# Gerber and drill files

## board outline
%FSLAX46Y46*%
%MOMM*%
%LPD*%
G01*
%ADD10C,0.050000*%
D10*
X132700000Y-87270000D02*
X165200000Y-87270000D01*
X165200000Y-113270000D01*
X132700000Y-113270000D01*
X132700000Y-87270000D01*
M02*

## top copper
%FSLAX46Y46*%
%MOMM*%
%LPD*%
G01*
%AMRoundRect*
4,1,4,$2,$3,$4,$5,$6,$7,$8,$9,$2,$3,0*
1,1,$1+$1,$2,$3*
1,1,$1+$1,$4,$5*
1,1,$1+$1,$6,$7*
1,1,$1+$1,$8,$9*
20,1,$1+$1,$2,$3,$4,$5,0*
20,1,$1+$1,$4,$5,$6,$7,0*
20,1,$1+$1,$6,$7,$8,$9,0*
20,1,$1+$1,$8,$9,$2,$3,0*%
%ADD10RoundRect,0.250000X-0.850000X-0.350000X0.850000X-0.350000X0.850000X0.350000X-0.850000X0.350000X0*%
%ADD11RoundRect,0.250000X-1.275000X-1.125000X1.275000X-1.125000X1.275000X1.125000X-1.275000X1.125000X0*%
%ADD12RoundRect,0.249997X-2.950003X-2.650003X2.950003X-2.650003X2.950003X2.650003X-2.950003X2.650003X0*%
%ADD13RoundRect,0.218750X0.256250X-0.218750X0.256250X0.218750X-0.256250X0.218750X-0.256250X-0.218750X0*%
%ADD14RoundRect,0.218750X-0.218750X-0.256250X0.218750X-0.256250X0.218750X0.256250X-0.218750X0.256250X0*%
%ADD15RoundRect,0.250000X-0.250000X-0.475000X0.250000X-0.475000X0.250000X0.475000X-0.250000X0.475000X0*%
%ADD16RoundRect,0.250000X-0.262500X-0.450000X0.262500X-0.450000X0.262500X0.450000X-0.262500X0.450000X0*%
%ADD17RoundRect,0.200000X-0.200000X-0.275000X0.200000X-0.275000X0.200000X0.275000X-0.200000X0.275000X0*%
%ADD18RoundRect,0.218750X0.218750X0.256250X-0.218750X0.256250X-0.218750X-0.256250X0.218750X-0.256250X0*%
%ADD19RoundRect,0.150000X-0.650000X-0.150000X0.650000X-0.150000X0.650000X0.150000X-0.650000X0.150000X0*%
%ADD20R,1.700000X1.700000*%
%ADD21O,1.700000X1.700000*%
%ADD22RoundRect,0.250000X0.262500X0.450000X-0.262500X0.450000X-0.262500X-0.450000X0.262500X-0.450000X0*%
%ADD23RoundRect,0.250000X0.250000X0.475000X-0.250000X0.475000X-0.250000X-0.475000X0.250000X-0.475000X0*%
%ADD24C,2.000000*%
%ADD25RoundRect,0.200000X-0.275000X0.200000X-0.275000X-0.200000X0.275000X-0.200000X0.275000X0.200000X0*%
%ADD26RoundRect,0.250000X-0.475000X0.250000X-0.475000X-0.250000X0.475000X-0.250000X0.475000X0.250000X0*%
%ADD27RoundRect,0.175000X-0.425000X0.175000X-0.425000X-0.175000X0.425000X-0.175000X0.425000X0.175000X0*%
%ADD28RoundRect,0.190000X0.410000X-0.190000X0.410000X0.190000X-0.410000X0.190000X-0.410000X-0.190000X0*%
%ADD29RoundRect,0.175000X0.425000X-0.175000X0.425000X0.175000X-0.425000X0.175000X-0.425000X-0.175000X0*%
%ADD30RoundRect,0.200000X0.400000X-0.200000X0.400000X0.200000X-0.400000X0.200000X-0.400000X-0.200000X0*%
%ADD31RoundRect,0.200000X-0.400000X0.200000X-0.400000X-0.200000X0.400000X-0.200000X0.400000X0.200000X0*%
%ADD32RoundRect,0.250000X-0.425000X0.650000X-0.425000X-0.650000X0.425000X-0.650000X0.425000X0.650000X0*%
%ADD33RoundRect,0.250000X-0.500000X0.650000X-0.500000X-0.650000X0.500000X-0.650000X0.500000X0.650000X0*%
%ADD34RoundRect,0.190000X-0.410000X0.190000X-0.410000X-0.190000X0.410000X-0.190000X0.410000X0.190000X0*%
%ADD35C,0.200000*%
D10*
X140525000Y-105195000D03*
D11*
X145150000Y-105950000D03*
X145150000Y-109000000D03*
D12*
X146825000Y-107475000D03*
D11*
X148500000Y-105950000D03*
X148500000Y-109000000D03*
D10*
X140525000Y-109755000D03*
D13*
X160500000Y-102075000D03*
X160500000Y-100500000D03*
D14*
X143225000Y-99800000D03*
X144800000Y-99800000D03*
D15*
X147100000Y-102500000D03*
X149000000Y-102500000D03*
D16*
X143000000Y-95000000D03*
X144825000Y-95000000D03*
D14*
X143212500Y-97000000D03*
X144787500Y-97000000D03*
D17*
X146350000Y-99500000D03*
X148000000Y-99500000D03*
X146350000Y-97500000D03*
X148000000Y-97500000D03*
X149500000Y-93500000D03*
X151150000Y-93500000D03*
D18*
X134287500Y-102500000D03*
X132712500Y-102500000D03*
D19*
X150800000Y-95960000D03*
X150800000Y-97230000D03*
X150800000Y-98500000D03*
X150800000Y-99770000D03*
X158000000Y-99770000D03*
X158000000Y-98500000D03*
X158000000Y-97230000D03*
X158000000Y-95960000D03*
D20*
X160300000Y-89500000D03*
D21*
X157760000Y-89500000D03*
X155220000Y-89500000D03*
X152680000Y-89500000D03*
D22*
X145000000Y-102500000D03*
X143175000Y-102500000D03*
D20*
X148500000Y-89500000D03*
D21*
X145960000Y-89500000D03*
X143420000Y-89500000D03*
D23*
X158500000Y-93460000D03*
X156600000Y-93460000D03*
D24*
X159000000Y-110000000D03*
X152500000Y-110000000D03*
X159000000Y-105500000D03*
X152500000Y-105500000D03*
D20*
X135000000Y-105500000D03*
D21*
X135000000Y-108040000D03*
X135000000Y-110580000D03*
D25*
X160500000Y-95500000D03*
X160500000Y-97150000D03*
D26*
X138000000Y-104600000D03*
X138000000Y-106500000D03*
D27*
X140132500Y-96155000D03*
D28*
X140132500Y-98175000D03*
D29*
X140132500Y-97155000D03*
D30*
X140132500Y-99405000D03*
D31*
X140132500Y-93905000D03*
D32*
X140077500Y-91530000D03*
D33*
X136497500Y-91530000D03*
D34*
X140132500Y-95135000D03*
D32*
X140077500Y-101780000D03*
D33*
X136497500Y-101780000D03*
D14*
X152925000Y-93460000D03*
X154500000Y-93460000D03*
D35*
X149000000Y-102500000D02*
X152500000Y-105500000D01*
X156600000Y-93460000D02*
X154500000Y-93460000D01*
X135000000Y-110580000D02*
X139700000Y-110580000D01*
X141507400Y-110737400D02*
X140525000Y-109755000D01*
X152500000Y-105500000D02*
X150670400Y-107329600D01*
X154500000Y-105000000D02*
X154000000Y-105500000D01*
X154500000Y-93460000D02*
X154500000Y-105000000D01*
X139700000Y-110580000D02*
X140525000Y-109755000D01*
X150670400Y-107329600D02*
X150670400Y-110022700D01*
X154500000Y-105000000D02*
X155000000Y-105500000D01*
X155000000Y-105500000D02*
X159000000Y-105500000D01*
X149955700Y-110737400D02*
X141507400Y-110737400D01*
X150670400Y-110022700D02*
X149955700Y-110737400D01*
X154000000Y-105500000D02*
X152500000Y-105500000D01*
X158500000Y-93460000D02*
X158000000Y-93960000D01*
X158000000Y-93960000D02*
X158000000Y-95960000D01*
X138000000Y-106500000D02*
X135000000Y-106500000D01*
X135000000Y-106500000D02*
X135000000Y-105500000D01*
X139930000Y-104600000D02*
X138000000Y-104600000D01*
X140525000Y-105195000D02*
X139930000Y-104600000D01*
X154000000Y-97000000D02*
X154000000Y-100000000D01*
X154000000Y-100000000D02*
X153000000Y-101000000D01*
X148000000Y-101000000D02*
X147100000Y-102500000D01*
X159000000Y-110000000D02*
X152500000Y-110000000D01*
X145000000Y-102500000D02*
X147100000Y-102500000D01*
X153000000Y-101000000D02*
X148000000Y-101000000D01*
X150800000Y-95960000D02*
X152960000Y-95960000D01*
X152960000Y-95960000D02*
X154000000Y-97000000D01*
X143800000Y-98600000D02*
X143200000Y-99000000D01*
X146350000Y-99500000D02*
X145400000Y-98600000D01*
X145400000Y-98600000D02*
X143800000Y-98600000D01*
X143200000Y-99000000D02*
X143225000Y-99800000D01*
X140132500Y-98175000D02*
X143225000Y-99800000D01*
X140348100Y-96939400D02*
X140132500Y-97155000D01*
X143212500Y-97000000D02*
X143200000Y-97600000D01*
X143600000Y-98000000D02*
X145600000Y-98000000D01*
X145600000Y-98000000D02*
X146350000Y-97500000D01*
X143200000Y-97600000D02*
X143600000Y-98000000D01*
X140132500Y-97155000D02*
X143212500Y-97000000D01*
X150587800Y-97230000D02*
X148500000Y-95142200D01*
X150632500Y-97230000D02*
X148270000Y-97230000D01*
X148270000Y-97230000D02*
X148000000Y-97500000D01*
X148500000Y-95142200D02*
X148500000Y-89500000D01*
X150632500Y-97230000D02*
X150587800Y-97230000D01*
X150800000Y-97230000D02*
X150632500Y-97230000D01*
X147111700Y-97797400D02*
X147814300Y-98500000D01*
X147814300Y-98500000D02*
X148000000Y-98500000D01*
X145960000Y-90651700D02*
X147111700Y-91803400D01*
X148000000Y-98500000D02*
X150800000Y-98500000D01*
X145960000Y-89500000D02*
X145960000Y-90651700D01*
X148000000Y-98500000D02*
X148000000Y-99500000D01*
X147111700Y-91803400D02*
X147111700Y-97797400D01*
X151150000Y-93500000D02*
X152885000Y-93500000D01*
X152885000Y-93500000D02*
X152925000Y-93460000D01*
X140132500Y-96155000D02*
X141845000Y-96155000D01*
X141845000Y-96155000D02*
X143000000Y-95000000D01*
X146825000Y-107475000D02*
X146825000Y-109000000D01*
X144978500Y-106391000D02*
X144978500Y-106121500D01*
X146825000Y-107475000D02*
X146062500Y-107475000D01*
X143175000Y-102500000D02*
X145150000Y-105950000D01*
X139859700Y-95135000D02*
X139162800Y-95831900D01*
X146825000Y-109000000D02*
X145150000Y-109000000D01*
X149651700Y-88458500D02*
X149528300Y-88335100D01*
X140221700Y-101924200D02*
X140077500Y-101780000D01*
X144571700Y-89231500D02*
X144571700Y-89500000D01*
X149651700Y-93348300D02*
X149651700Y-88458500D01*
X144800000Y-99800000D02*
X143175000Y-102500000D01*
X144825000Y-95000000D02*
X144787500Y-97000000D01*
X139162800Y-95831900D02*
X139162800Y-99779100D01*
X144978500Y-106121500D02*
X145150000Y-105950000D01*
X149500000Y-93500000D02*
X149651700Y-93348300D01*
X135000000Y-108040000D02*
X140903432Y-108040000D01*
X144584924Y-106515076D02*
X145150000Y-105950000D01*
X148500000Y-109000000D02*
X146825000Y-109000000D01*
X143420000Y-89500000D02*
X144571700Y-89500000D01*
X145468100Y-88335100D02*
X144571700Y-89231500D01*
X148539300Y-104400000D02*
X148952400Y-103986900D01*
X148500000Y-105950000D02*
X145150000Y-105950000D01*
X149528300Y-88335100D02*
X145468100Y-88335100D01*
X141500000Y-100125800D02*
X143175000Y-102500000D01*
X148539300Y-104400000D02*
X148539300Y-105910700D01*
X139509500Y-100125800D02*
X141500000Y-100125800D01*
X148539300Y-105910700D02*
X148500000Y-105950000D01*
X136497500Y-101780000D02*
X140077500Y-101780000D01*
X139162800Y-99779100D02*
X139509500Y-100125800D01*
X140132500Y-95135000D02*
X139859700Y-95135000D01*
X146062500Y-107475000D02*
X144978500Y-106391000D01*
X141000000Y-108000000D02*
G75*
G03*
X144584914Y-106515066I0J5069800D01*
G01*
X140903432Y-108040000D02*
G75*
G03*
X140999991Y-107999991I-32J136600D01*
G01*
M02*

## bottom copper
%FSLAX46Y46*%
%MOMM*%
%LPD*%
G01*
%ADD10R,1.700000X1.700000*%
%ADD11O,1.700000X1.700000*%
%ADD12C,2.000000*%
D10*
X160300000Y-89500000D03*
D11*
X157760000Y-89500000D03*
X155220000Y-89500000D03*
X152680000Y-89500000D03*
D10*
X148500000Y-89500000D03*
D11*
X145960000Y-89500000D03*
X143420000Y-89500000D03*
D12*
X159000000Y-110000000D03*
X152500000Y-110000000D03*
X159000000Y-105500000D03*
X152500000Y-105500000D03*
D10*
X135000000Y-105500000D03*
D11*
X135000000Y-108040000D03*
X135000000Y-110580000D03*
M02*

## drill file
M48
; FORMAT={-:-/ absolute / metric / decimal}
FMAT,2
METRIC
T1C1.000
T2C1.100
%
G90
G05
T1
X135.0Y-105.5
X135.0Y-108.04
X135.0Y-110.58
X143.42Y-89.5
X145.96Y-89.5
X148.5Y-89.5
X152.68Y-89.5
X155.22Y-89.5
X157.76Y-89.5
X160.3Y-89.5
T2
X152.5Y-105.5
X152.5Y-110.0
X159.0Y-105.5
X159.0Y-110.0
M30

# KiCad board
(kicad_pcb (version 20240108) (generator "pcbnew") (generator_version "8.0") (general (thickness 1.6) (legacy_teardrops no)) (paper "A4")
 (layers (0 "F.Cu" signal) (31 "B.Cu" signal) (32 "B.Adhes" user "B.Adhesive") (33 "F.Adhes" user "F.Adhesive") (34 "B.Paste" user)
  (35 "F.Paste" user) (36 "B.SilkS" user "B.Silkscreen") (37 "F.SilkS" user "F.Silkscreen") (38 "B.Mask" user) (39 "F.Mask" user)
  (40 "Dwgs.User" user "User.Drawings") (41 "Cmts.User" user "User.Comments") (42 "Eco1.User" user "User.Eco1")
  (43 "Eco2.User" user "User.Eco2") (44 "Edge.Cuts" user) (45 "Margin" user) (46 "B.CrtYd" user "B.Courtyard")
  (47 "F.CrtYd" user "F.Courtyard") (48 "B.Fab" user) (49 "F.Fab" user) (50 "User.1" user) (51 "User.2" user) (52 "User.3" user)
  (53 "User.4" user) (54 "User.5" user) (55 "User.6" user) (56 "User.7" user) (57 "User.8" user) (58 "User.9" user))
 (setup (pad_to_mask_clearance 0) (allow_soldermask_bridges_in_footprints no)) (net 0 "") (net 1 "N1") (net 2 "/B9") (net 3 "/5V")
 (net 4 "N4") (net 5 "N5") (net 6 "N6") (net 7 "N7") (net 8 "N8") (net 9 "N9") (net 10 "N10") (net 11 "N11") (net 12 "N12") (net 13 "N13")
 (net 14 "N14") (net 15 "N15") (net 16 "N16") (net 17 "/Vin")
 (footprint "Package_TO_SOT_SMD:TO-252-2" (layer "F.Cu") (at 145.565 107.475)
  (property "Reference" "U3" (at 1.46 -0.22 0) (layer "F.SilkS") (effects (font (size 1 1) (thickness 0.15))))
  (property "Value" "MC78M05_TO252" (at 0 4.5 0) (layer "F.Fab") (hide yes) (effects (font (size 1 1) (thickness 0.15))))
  (pad "1" smd roundrect (at -5.04 -2.28) (size 2.2 1.2) (layers "F.Cu" "F.Paste" "F.Mask") (roundrect_rratio 0.208333) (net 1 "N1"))
  (pad "2" smd roundrect (at -0.415 -1.525) (size 3.05 2.75) (layers "F.Cu" "F.Paste") (roundrect_rratio 0.090909) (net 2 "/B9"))
  (pad "2" smd roundrect (at -0.415 1.525) (size 3.05 2.75) (layers "F.Cu" "F.Paste") (roundrect_rratio 0.090909) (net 2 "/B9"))
  (pad "2" smd roundrect (at 1.26 0) (size 6.4 5.8) (layers "F.Cu" "F.Mask") (roundrect_rratio 0.043103) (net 2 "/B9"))
  (pad "2" smd roundrect (at 2.935 -1.525) (size 3.05 2.75) (layers "F.Cu" "F.Paste") (roundrect_rratio 0.090909) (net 2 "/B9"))
  (pad "2" smd roundrect (at 2.935 1.525) (size 3.05 2.75) (layers "F.Cu" "F.Paste") (roundrect_rratio 0.090909) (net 2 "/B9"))
  (pad "3" smd roundrect (at -5.04 2.28) (size 2.2 1.2) (layers "F.Cu" "F.Paste" "F.Mask") (roundrect_rratio 0.208333) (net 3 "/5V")))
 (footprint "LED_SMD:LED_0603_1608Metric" (layer "F.Cu") (at 160.5 101.2875 90)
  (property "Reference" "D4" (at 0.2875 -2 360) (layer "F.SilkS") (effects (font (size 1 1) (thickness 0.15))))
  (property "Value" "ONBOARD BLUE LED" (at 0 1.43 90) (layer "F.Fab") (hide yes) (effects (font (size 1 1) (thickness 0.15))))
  (pad "1" smd roundrect (at -0.7875 0 90) (size 0.875 0.95) (layers "F.Cu" "F.Paste" "F.Mask") (roundrect_rratio 0.25) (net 2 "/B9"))
  (pad "2" smd roundrect (at 0.7875 0 90) (size 0.875 0.95) (layers "F.Cu" "F.Paste" "F.Mask") (roundrect_rratio 0.25) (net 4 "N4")))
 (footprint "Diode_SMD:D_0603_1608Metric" (layer "F.Cu") (at 144.0125 99.8)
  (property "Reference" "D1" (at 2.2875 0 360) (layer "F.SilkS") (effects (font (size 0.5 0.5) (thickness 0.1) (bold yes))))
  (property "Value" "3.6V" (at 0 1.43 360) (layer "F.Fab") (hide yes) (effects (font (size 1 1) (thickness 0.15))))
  (pad "1" smd roundrect (at -0.7875 0) (size 0.875 0.95) (layers "F.Cu" "F.Paste" "F.Mask") (roundrect_rratio 0.25) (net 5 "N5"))
  (pad "2" smd roundrect (at 0.7875 0) (size 0.875 0.95) (layers "F.Cu" "F.Paste" "F.Mask") (roundrect_rratio 0.25) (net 2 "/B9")))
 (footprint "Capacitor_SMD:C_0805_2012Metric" (layer "F.Cu") (at 148.05 102.5)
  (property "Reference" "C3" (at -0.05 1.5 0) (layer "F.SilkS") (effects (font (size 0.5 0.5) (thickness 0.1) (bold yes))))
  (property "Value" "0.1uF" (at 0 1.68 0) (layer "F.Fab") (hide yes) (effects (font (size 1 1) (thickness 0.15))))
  (pad "1" smd roundrect (at -0.95 0) (size 1 1.45) (layers "F.Cu" "F.Paste" "F.Mask") (roundrect_rratio 0.25) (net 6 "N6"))
  (pad "2" smd roundrect (at 0.95 0) (size 1 1.45) (layers "F.Cu" "F.Paste" "F.Mask") (roundrect_rratio 0.25) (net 3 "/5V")))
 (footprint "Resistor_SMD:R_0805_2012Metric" (layer "F.Cu") (at 143.9125 95)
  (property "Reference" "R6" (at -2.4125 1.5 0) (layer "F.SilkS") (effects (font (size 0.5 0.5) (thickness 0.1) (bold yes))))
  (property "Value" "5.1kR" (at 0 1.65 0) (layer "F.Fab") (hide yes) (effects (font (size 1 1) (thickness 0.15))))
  (pad "1" smd roundrect (at -0.9125 0) (size 1.025 1.4) (layers "F.Cu" "F.Paste" "F.Mask") (roundrect_rratio 0.243902) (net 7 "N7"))
  (pad "2" smd roundrect (at 0.9125 0) (size 1.025 1.4) (layers "F.Cu" "F.Paste" "F.Mask") (roundrect_rratio 0.243902) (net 2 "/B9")))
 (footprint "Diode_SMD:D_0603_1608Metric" (layer "F.Cu") (at 144 97)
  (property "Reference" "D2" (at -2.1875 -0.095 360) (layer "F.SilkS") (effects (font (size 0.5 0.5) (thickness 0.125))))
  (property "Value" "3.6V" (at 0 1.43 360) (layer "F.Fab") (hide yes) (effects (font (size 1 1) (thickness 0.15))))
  (pad "1" smd roundrect (at -0.7875 0) (size 0.875 0.95) (layers "F.Cu" "F.Paste" "F.Mask") (roundrect_rratio 0.25) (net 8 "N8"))
  (pad "2" smd roundrect (at 0.7875 0) (size 0.875 0.95) (layers "F.Cu" "F.Paste" "F.Mask") (roundrect_rratio 0.25) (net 2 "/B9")))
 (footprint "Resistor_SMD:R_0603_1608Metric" (layer "F.Cu") (at 147.175 99.5)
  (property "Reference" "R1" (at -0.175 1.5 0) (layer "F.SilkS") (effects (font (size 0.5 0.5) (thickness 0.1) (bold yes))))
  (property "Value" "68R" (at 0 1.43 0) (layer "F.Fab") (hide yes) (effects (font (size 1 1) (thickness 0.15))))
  (pad "1" smd roundrect (at -0.825 0) (size 0.8 0.95) (layers "F.Cu" "F.Paste" "F.Mask") (roundrect_rratio 0.25) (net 5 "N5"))
  (pad "2" smd roundrect (at 0.825 0) (size 0.8 0.95) (layers "F.Cu" "F.Paste" "F.Mask") (roundrect_rratio 0.25) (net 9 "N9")))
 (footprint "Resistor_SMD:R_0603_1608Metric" (layer "F.Cu") (at 147.175 97.5)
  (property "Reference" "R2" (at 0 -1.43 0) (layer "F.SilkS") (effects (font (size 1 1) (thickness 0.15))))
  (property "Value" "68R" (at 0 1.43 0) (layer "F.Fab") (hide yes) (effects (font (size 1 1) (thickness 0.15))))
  (pad "1" smd roundrect (at -0.825 0) (size 0.8 0.95) (layers "F.Cu" "F.Paste" "F.Mask") (roundrect_rratio 0.25) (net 8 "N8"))
  (pad "2" smd roundrect (at 0.825 0) (size 0.8 0.95) (layers "F.Cu" "F.Paste" "F.Mask") (roundrect_rratio 0.25) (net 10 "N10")))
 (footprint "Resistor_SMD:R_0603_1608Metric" (layer "F.Cu") (at 150.325 93.5)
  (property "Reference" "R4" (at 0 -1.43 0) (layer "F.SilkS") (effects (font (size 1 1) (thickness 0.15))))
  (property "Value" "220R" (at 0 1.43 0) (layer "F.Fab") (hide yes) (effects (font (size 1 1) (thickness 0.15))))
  (pad "1" smd roundrect (at -0.825 0) (size 0.8 0.95) (layers "F.Cu" "F.Paste" "F.Mask") (roundrect_rratio 0.25) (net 2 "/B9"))
  (pad "2" smd roundrect (at 0.825 0) (size 0.8 0.95) (layers "F.Cu" "F.Paste" "F.Mask") (roundrect_rratio 0.25) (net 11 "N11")))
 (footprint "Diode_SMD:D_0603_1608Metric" (layer "F.Cu") (at 133.5 102.5 180)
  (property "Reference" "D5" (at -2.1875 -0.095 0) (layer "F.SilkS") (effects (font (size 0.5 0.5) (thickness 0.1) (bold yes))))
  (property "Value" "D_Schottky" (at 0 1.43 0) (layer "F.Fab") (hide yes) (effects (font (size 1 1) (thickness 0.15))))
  (pad "1" smd roundrect (at -0.7875 0 180) (size 0.875 0.95) (layers "F.Cu" "F.Paste" "F.Mask") (roundrect_rratio 0.25) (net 1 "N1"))
  (pad "2" smd roundrect (at 0.7875 0 180) (size 0.875 0.95) (layers "F.Cu" "F.Paste" "F.Mask") (roundrect_rratio 0.25) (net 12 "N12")))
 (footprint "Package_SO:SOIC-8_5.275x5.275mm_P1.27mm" (layer "F.Cu") (at 154.4 97.865)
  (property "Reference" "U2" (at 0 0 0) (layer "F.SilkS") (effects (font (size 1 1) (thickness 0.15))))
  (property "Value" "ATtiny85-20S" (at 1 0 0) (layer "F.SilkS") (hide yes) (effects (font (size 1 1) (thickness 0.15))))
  (pad "1" smd roundrect (at -3.6 -1.905) (size 1.6 0.6) (layers "F.Cu" "F.Paste" "F.Mask") (roundrect_rratio 0.25) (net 6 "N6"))
  (pad "2" smd roundrect (at -3.6 -0.635) (size 1.6 0.6) (layers "F.Cu" "F.Paste" "F.Mask") (roundrect_rratio 0.25) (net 10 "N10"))
  (pad "3" smd roundrect (at -3.6 0.635) (size 1.6 0.6) (layers "F.Cu" "F.Paste" "F.Mask") (roundrect_rratio 0.25) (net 9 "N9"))
  (pad "4" smd roundrect (at -3.6 1.905) (size 1.6 0.6) (layers "F.Cu" "F.Paste" "F.Mask") (roundrect_rratio 0.25) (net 2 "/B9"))
  (pad "5" smd roundrect (at 3.6 1.905) (size 1.6 0.6) (layers "F.Cu" "F.Paste" "F.Mask") (roundrect_rratio 0.25) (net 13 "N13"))
  (pad "6" smd roundrect (at 3.6 0.635) (size 1.6 0.6) (layers "F.Cu" "F.Paste" "F.Mask") (roundrect_rratio 0.25) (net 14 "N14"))
  (pad "7" smd roundrect (at 3.6 -0.635) (size 1.6 0.6) (layers "F.Cu" "F.Paste" "F.Mask") (roundrect_rratio 0.25) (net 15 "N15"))
  (pad "8" smd roundrect (at 3.6 -1.905) (size 1.6 0.6) (layers "F.Cu" "F.Paste" "F.Mask") (roundrect_rratio 0.25) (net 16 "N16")))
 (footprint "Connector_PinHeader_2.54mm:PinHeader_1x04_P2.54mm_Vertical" (layer "F.Cu") (at 160.3 89.5 -90)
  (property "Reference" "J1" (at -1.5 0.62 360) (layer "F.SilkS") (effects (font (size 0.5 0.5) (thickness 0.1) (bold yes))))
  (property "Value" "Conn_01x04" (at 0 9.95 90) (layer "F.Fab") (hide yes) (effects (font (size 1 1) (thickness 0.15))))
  (pad "1" thru_hole rect (at 0 0 270) (size 1.7 1.7) (drill 1) (layers "*.Cu" "*.Mask") (remove_unused_layers no) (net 13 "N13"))
  (pad "2" thru_hole oval (at 0 2.54 270) (size 1.7 1.7) (drill 1) (layers "*.Cu" "*.Mask") (remove_unused_layers no) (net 14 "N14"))
  (pad "3" thru_hole oval (at 0 5.08 270) (size 1.7 1.7) (drill 1) (layers "*.Cu" "*.Mask") (remove_unused_layers no) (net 15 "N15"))
  (pad "4" thru_hole oval (at 0 7.62 270) (size 1.7 1.7) (drill 1) (layers "*.Cu" "*.Mask") (remove_unused_layers no) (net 2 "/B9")))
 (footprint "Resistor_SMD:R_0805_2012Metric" (layer "F.Cu") (at 144.0875 102.5 180)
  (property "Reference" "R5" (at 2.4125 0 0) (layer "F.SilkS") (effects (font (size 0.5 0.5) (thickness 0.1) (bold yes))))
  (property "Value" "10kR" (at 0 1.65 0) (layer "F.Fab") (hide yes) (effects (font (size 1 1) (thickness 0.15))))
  (pad "1" smd roundrect (at -0.9125 0 180) (size 1.025 1.4) (layers "F.Cu" "F.Paste" "F.Mask") (roundrect_rratio 0.243902) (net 6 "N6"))
  (pad "2" smd roundrect (at 0.9125 0 180) (size 1.025 1.4) (layers "F.Cu" "F.Paste" "F.Mask") (roundrect_rratio 0.243902) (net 2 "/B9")))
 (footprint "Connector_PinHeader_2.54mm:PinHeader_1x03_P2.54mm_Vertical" (layer "F.Cu") (at 148.5 89.5 -90)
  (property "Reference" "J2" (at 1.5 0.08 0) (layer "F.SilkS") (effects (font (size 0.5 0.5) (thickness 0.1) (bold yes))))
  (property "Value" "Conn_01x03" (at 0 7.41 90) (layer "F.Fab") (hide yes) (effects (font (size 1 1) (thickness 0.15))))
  (pad "1" thru_hole rect (at 0 0 270) (size 1.7 1.7) (drill 1) (layers "*.Cu" "*.Mask") (remove_unused_layers no) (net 10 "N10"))
  (pad "2" thru_hole oval (at 0 2.54 270) (size 1.7 1.7) (drill 1) (layers "*.Cu" "*.Mask") (remove_unused_layers no) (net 9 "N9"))
  (pad "3" thru_hole oval (at 0 5.08 270) (size 1.7 1.7) (drill 1) (layers "*.Cu" "*.Mask") (remove_unused_layers no) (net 2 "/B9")))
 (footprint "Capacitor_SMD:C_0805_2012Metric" (layer "F.Cu") (at 157.55 93.46 180)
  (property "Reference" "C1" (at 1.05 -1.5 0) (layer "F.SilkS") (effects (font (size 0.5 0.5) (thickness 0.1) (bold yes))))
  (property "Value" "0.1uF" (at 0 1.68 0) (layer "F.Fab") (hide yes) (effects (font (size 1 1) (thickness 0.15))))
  (pad "1" smd roundrect (at -0.95 0 180) (size 1 1.45) (layers "F.Cu" "F.Paste" "F.Mask") (roundrect_rratio 0.25) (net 16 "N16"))
  (pad "2" smd roundrect (at 0.95 0 180) (size 1 1.45) (layers "F.Cu" "F.Paste" "F.Mask") (roundrect_rratio 0.25) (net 3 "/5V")))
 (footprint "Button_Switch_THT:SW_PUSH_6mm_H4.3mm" (layer "F.Cu") (at 159 110 180)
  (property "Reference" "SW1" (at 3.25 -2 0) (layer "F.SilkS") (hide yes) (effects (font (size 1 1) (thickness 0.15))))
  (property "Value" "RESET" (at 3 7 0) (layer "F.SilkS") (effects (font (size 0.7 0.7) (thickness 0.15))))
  (pad "1" thru_hole circle (at 0 0 270) (size 2 2) (drill 1.1) (layers "*.Cu" "*.Mask") (remove_unused_layers no) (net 6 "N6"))
  (pad "1" thru_hole circle (at 6.5 0 270) (size 2 2) (drill 1.1) (layers "*.Cu" "*.Mask") (remove_unused_layers no) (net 6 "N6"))
  (pad "2" thru_hole circle (at 0 4.5 270) (size 2 2) (drill 1.1) (layers "*.Cu" "*.Mask") (remove_unused_layers no) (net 3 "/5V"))
  (pad "2" thru_hole circle (at 6.5 4.5 270) (size 2 2) (drill 1.1) (layers "*.Cu" "*.Mask") (remove_unused_layers no) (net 3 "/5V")))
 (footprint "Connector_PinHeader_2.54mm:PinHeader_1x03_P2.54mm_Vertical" (layer "F.Cu") (at 135 105.5)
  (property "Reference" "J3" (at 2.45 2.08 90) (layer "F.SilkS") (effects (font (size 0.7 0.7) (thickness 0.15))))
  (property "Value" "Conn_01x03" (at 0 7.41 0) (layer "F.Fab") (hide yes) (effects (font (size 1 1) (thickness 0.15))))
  (pad "1" thru_hole rect (at 0 0) (size 1.7 1.7) (drill 1) (layers "*.Cu" "*.Mask") (remove_unused_layers no) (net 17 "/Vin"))
  (pad "2" thru_hole oval (at 0 2.54) (size 1.7 1.7) (drill 1) (layers "*.Cu" "*.Mask") (remove_unused_layers no) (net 2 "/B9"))
  (pad "3" thru_hole oval (at 0 5.08) (size 1.7 1.7) (drill 1) (layers "*.Cu" "*.Mask") (remove_unused_layers no) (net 3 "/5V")))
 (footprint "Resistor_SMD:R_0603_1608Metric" (layer "F.Cu") (at 160.5 96.325 -90)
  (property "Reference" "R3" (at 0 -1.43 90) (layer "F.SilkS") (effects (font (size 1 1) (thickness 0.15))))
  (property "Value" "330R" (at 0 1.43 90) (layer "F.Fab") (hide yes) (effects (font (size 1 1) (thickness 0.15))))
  (pad "1" smd roundrect (at -0.825 0 270) (size 0.8 0.95) (layers "F.Cu" "F.Paste" "F.Mask") (roundrect_rratio 0.25) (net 13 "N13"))
  (pad "2" smd roundrect (at 0.825 0 270) (size 0.8 0.95) (layers "F.Cu" "F.Paste" "F.Mask") (roundrect_rratio 0.25) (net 4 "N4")))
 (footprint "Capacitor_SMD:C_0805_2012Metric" (layer "F.Cu") (at 138 105.55 -90)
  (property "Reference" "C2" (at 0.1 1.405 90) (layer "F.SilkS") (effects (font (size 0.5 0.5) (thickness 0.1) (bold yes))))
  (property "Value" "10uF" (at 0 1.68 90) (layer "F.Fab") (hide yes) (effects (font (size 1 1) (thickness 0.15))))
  (pad "1" smd roundrect (at -0.95 0 270) (size 1 1.45) (layers "F.Cu" "F.Paste" "F.Mask") (roundrect_rratio 0.25) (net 1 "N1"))
  (pad "2" smd roundrect (at 0.95 0 270) (size 1 1.45) (layers "F.Cu" "F.Paste" "F.Mask") (roundrect_rratio 0.25) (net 17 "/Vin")))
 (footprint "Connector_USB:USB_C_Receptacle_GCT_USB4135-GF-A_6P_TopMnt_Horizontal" (layer "F.Cu") (at 137.1 96.655 -90)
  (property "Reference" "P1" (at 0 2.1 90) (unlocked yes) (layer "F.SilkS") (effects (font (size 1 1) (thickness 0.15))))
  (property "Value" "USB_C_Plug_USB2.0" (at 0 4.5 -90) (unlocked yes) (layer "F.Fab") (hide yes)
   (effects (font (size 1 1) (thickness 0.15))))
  (pad "A5" smd roundrect (at -0.5 -3.0325 270) (size 0.7 1.2) (layers "F.Cu" "F.Paste" "F.Mask") (roundrect_rratio 0.25) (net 7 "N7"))
  (pad "A6" smd roundrect (at 1.52 -3.0325 90) (size 0.76 1.2) (layers "F.Cu" "F.Paste" "F.Mask") (roundrect_rratio 0.25) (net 5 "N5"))
  (pad "A7" smd roundrect (at 0.5 -3.0325 90) (size 0.7 1.2) (layers "F.Cu" "F.Paste" "F.Mask") (roundrect_rratio 0.25) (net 8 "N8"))
  (pad "A12" smd roundrect (at 2.75 -3.0325 90) (size 0.8 1.2) (layers "F.Cu" "F.Paste" "F.Mask") (roundrect_rratio 0.25))
  (pad "B5" smd roundrect (at -2.75 -3.0325 270) (size 0.8 1.2) (layers "F.Cu" "F.Paste" "F.Mask") (roundrect_rratio 0.25) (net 12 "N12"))
  (pad "S1" smd roundrect (at -5.125 -2.9775 270) (size 1.8 1.35) (layers "F.Cu" "F.Paste" "F.Mask") (roundrect_rratio 0.1851851852)
   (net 2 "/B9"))
  (pad "S1" smd roundrect (at -5.125 0.6025 270) (size 1.8 1.5) (layers "F.Cu" "F.Paste" "F.Mask") (roundrect_rratio 0.1666666667)
   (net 2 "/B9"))
  (pad "S1" smd roundrect (at -1.52 -3.0325 270) (size 0.76 1.2) (layers "F.Cu" "F.Paste" "F.Mask") (roundrect_rratio 0.25) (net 2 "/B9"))
  (pad "S1" smd roundrect (at 5.125 -2.9775 270) (size 1.8 1.35) (layers "F.Cu" "F.Paste" "F.Mask") (roundrect_rratio 0.1851851852)
   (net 2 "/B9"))
  (pad "S1" smd roundrect (at 5.125 0.6025 270) (size 1.8 1.5) (layers "F.Cu" "F.Paste" "F.Mask") (roundrect_rratio 0.1666666667)
   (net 2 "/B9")))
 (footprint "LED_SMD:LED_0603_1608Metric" (layer "F.Cu") (at 153.7125 93.46)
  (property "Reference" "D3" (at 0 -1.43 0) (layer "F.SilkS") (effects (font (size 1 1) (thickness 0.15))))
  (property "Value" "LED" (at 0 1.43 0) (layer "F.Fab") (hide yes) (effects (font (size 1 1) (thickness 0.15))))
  (pad "1" smd roundrect (at -0.7875 0) (size 0.875 0.95) (layers "F.Cu" "F.Paste" "F.Mask") (roundrect_rratio 0.25) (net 11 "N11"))
  (pad "2" smd roundrect (at 0.7875 0) (size 0.875 0.95) (layers "F.Cu" "F.Paste" "F.Mask") (roundrect_rratio 0.25) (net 3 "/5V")))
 (gr_rect (start 132.7 87.27) (end 165.2 113.27) (stroke (width 0.05) (type default)) (fill none) (layer "Edge.Cuts"))
 (segment (start 149 102.5) (end 152.5 105.5) (width 0.2) (layer "F.Cu") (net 3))
 (segment (start 156.6 93.46) (end 154.5 93.46) (width 0.2) (layer "F.Cu") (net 3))
 (segment (start 135 110.58) (end 139.7 110.58) (width 0.2) (layer "F.Cu") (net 3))
 (segment (start 141.5074 110.7374) (end 140.525 109.755) (width 0.2) (layer "F.Cu") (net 3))
 (segment (start 152.5 105.5) (end 150.6704 107.3296) (width 0.2) (layer "F.Cu") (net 3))
 (segment (start 154.5 105) (end 154 105.5) (width 0.2) (layer "F.Cu") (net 3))
 (segment (start 154.5 93.46) (end 154.5 105) (width 0.2) (layer "F.Cu") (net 3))
 (segment (start 139.7 110.58) (end 140.525 109.755) (width 0.2) (layer "F.Cu") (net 3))
 (segment (start 150.6704 107.3296) (end 150.6704 110.0227) (width 0.2) (layer "F.Cu") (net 3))
 (segment (start 154.5 105) (end 155 105.5) (width 0.2) (layer "F.Cu") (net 3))
 (segment (start 155 105.5) (end 159 105.5) (width 0.2) (layer "F.Cu") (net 3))
 (segment (start 149.9557 110.7374) (end 141.5074 110.7374) (width 0.2) (layer "F.Cu") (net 3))
 (segment (start 150.6704 110.0227) (end 149.9557 110.7374) (width 0.2) (layer "F.Cu") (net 3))
 (segment (start 154 105.5) (end 152.5 105.5) (width 0.2) (layer "F.Cu") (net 3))
 (segment (start 158.5 93.46) (end 158 93.96) (width 0.2) (layer "F.Cu") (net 16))
 (segment (start 158 93.96) (end 158 95.96) (width 0.2) (layer "F.Cu") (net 16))
 (segment (start 138 106.5) (end 135 106.5) (width 0.2) (layer "F.Cu") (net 17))
 (segment (start 135 106.5) (end 135 105.5) (width 0.2) (layer "F.Cu") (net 17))
 (segment (start 139.93 104.6) (end 138 104.6) (width 0.2) (layer "F.Cu") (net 1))
 (segment (start 140.525 105.195) (end 139.93 104.6) (width 0.2) (layer "F.Cu") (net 1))
 (segment (start 154 97) (end 154 100) (width 0.2) (layer "F.Cu") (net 6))
 (segment (start 154 100) (end 153 101) (width 0.2) (layer "F.Cu") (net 6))
 (segment (start 148 101) (end 147.1 102.5) (width 0.2) (layer "F.Cu") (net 6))
 (segment (start 159 110) (end 152.5 110) (width 0.2) (layer "F.Cu") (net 6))
 (segment (start 145 102.5) (end 147.1 102.5) (width 0.2) (layer "F.Cu") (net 6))
 (segment (start 153 101) (end 148 101) (width 0.2) (layer "F.Cu") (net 6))
 (segment (start 150.8 95.96) (end 152.96 95.96) (width 0.2) (layer "F.Cu") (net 6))
 (segment (start 152.96 95.96) (end 154 97) (width 0.2) (layer "F.Cu") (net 6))
 (segment (start 143.8 98.6) (end 143.2 99) (width 0.2) (layer "F.Cu") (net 5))
 (segment (start 146.35 99.5) (end 145.4 98.6) (width 0.2) (layer "F.Cu") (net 5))
 (segment (start 145.4 98.6) (end 143.8 98.6) (width 0.2) (layer "F.Cu") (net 5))
 (segment (start 143.2 99) (end 143.225 99.8) (width 0.2) (layer "F.Cu") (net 5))
 (segment (start 140.1325 98.175) (end 143.225 99.8) (width 0.2) (layer "F.Cu") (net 5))
 (segment (start 140.3481 96.9394) (end 140.1325 97.155) (width 0.2) (layer "F.Cu") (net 8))
 (segment (start 143.2125 97) (end 143.2 97.6) (width 0.2) (layer "F.Cu") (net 8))
 (segment (start 143.6 98) (end 145.6 98) (width 0.2) (layer "F.Cu") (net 8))
 (segment (start 145.6 98) (end 146.35 97.5) (width 0.2) (layer "F.Cu") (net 8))
 (segment (start 143.2 97.6) (end 143.6 98) (width 0.2) (layer "F.Cu") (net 8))
 (segment (start 140.1325 97.155) (end 143.2125 97) (width 0.2) (layer "F.Cu") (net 8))
 (segment (start 150.5878 97.23) (end 148.5 95.1422) (width 0.2) (layer "F.Cu") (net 10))
 (segment (start 150.6325 97.23) (end 148.27 97.23) (width 0.2) (layer "F.Cu") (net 10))
 (segment (start 148.27 97.23) (end 148 97.5) (width 0.2) (layer "F.Cu") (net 10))
 (segment (start 148.5 95.1422) (end 148.5 89.5) (width 0.2) (layer "F.Cu") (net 10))
 (segment (start 150.6325 97.23) (end 150.5878 97.23) (width 0.2) (layer "F.Cu") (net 10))
 (segment (start 150.8 97.23) (end 150.6325 97.23) (width 0.2) (layer "F.Cu") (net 10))
 (segment (start 147.1117 97.7974) (end 147.8143 98.5) (width 0.2) (layer "F.Cu") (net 9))
 (segment (start 147.8143 98.5) (end 148 98.5) (width 0.2) (layer "F.Cu") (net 9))
 (segment (start 145.96 90.6517) (end 147.1117 91.8034) (width 0.2) (layer "F.Cu") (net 9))
 (segment (start 148 98.5) (end 150.8 98.5) (width 0.2) (layer "F.Cu") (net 9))
 (segment (start 145.96 89.5) (end 145.96 90.6517) (width 0.2) (layer "F.Cu") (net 9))
 (segment (start 148 98.5) (end 148 99.5) (width 0.2) (layer "F.Cu") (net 9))
 (segment (start 147.1117 91.8034) (end 147.1117 97.7974) (width 0.2) (layer "F.Cu") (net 9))
 (segment (start 151.15 93.5) (end 152.885 93.5) (width 0.2) (layer "F.Cu") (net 11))
 (segment (start 152.885 93.5) (end 152.925 93.46) (width 0.2) (layer "F.Cu") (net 11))
 (segment (start 140.1325 96.155) (end 141.845 96.155) (width 0.2) (layer "F.Cu") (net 7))
 (segment (start 141.845 96.155) (end 143 95) (width 0.2) (layer "F.Cu") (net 7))
 (segment (start 146.825 107.475) (end 146.825 109) (width 0.2) (layer "F.Cu") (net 2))
 (segment (start 144.9785 106.391) (end 144.9785 106.1215) (width 0.2) (layer "F.Cu") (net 2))
 (segment (start 146.825 107.475) (end 146.0625 107.475) (width 0.2) (layer "F.Cu") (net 2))
 (segment (start 143.175 102.5) (end 145.15 105.95) (width 0.2) (layer "F.Cu") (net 2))
 (segment (start 139.8597 95.135) (end 139.1628 95.8319) (width 0.2) (layer "F.Cu") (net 2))
 (segment (start 146.825 109) (end 145.15 109) (width 0.2) (layer "F.Cu") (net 2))
 (segment (start 149.6517 88.4585) (end 149.5283 88.3351) (width 0.2) (layer "F.Cu") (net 2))
 (segment (start 140.2217 101.9242) (end 140.0775 101.78) (width 0.2) (layer "F.Cu") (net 2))
 (segment (start 144.5717 89.2315) (end 144.5717 89.5) (width 0.2) (layer "F.Cu") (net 2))
 (segment (start 149.6517 93.3483) (end 149.6517 88.4585) (width 0.2) (layer "F.Cu") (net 2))
 (segment (start 144.8 99.8) (end 143.175 102.5) (width 0.2) (layer "F.Cu") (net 2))
 (segment (start 144.825 95) (end 144.7875 97) (width 0.2) (layer "F.Cu") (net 2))
 (segment (start 139.1628 95.8319) (end 139.1628 99.7791) (width 0.2) (layer "F.Cu") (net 2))
 (segment (start 144.9785 106.1215) (end 145.15 105.95) (width 0.2) (layer "F.Cu") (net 2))
 (segment (start 149.5 93.5) (end 149.6517 93.3483) (width 0.2) (layer "F.Cu") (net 2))
 (segment (start 135 108.04) (end 140.903432 108.04) (width 0.2) (layer "F.Cu") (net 2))
 (segment (start 144.584924 106.515076) (end 145.15 105.95) (width 0.2) (layer "F.Cu") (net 2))
 (segment (start 148.5 109) (end 146.825 109) (width 0.2) (layer "F.Cu") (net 2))
 (segment (start 143.42 89.5) (end 144.5717 89.5) (width 0.2) (layer "F.Cu") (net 2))
 (segment (start 145.4681 88.3351) (end 144.5717 89.2315) (width 0.2) (layer "F.Cu") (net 2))
 (segment (start 148.5393 104.4) (end 148.9524 103.9869) (width 0.2) (layer "F.Cu") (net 2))
 (segment (start 148.5 105.95) (end 145.15 105.95) (width 0.2) (layer "F.Cu") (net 2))
 (segment (start 149.5283 88.3351) (end 145.4681 88.3351) (width 0.2) (layer "F.Cu") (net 2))
 (segment (start 141.5 100.1258) (end 143.175 102.5) (width 0.2) (layer "F.Cu") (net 2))
 (segment (start 148.5393 104.4) (end 148.5393 105.9107) (width 0.2) (layer "F.Cu") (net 2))
 (segment (start 139.5095 100.1258) (end 141.5 100.1258) (width 0.2) (layer "F.Cu") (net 2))
 (segment (start 148.5393 105.9107) (end 148.5 105.95) (width 0.2) (layer "F.Cu") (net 2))
 (segment (start 136.4975 101.78) (end 140.0775 101.78) (width 0.2) (layer "F.Cu") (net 2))
 (segment (start 139.1628 99.7791) (end 139.5095 100.1258) (width 0.2) (layer "F.Cu") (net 2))
 (segment (start 140.1325 95.135) (end 139.8597 95.135) (width 0.2) (layer "F.Cu") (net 2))
 (segment (start 146.0625 107.475) (end 144.9785 106.391) (width 0.2) (layer "F.Cu") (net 2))
 (arc (start 141 108) (mid 142.940147 107.614081) (end 144.584924 106.515076) (width 0.2) (layer "F.Cu") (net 2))
 (arc (start 140.903432 108.04) (mid 140.955694 108.029604) (end 141 108) (width 0.2) (layer "F.Cu") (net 2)))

